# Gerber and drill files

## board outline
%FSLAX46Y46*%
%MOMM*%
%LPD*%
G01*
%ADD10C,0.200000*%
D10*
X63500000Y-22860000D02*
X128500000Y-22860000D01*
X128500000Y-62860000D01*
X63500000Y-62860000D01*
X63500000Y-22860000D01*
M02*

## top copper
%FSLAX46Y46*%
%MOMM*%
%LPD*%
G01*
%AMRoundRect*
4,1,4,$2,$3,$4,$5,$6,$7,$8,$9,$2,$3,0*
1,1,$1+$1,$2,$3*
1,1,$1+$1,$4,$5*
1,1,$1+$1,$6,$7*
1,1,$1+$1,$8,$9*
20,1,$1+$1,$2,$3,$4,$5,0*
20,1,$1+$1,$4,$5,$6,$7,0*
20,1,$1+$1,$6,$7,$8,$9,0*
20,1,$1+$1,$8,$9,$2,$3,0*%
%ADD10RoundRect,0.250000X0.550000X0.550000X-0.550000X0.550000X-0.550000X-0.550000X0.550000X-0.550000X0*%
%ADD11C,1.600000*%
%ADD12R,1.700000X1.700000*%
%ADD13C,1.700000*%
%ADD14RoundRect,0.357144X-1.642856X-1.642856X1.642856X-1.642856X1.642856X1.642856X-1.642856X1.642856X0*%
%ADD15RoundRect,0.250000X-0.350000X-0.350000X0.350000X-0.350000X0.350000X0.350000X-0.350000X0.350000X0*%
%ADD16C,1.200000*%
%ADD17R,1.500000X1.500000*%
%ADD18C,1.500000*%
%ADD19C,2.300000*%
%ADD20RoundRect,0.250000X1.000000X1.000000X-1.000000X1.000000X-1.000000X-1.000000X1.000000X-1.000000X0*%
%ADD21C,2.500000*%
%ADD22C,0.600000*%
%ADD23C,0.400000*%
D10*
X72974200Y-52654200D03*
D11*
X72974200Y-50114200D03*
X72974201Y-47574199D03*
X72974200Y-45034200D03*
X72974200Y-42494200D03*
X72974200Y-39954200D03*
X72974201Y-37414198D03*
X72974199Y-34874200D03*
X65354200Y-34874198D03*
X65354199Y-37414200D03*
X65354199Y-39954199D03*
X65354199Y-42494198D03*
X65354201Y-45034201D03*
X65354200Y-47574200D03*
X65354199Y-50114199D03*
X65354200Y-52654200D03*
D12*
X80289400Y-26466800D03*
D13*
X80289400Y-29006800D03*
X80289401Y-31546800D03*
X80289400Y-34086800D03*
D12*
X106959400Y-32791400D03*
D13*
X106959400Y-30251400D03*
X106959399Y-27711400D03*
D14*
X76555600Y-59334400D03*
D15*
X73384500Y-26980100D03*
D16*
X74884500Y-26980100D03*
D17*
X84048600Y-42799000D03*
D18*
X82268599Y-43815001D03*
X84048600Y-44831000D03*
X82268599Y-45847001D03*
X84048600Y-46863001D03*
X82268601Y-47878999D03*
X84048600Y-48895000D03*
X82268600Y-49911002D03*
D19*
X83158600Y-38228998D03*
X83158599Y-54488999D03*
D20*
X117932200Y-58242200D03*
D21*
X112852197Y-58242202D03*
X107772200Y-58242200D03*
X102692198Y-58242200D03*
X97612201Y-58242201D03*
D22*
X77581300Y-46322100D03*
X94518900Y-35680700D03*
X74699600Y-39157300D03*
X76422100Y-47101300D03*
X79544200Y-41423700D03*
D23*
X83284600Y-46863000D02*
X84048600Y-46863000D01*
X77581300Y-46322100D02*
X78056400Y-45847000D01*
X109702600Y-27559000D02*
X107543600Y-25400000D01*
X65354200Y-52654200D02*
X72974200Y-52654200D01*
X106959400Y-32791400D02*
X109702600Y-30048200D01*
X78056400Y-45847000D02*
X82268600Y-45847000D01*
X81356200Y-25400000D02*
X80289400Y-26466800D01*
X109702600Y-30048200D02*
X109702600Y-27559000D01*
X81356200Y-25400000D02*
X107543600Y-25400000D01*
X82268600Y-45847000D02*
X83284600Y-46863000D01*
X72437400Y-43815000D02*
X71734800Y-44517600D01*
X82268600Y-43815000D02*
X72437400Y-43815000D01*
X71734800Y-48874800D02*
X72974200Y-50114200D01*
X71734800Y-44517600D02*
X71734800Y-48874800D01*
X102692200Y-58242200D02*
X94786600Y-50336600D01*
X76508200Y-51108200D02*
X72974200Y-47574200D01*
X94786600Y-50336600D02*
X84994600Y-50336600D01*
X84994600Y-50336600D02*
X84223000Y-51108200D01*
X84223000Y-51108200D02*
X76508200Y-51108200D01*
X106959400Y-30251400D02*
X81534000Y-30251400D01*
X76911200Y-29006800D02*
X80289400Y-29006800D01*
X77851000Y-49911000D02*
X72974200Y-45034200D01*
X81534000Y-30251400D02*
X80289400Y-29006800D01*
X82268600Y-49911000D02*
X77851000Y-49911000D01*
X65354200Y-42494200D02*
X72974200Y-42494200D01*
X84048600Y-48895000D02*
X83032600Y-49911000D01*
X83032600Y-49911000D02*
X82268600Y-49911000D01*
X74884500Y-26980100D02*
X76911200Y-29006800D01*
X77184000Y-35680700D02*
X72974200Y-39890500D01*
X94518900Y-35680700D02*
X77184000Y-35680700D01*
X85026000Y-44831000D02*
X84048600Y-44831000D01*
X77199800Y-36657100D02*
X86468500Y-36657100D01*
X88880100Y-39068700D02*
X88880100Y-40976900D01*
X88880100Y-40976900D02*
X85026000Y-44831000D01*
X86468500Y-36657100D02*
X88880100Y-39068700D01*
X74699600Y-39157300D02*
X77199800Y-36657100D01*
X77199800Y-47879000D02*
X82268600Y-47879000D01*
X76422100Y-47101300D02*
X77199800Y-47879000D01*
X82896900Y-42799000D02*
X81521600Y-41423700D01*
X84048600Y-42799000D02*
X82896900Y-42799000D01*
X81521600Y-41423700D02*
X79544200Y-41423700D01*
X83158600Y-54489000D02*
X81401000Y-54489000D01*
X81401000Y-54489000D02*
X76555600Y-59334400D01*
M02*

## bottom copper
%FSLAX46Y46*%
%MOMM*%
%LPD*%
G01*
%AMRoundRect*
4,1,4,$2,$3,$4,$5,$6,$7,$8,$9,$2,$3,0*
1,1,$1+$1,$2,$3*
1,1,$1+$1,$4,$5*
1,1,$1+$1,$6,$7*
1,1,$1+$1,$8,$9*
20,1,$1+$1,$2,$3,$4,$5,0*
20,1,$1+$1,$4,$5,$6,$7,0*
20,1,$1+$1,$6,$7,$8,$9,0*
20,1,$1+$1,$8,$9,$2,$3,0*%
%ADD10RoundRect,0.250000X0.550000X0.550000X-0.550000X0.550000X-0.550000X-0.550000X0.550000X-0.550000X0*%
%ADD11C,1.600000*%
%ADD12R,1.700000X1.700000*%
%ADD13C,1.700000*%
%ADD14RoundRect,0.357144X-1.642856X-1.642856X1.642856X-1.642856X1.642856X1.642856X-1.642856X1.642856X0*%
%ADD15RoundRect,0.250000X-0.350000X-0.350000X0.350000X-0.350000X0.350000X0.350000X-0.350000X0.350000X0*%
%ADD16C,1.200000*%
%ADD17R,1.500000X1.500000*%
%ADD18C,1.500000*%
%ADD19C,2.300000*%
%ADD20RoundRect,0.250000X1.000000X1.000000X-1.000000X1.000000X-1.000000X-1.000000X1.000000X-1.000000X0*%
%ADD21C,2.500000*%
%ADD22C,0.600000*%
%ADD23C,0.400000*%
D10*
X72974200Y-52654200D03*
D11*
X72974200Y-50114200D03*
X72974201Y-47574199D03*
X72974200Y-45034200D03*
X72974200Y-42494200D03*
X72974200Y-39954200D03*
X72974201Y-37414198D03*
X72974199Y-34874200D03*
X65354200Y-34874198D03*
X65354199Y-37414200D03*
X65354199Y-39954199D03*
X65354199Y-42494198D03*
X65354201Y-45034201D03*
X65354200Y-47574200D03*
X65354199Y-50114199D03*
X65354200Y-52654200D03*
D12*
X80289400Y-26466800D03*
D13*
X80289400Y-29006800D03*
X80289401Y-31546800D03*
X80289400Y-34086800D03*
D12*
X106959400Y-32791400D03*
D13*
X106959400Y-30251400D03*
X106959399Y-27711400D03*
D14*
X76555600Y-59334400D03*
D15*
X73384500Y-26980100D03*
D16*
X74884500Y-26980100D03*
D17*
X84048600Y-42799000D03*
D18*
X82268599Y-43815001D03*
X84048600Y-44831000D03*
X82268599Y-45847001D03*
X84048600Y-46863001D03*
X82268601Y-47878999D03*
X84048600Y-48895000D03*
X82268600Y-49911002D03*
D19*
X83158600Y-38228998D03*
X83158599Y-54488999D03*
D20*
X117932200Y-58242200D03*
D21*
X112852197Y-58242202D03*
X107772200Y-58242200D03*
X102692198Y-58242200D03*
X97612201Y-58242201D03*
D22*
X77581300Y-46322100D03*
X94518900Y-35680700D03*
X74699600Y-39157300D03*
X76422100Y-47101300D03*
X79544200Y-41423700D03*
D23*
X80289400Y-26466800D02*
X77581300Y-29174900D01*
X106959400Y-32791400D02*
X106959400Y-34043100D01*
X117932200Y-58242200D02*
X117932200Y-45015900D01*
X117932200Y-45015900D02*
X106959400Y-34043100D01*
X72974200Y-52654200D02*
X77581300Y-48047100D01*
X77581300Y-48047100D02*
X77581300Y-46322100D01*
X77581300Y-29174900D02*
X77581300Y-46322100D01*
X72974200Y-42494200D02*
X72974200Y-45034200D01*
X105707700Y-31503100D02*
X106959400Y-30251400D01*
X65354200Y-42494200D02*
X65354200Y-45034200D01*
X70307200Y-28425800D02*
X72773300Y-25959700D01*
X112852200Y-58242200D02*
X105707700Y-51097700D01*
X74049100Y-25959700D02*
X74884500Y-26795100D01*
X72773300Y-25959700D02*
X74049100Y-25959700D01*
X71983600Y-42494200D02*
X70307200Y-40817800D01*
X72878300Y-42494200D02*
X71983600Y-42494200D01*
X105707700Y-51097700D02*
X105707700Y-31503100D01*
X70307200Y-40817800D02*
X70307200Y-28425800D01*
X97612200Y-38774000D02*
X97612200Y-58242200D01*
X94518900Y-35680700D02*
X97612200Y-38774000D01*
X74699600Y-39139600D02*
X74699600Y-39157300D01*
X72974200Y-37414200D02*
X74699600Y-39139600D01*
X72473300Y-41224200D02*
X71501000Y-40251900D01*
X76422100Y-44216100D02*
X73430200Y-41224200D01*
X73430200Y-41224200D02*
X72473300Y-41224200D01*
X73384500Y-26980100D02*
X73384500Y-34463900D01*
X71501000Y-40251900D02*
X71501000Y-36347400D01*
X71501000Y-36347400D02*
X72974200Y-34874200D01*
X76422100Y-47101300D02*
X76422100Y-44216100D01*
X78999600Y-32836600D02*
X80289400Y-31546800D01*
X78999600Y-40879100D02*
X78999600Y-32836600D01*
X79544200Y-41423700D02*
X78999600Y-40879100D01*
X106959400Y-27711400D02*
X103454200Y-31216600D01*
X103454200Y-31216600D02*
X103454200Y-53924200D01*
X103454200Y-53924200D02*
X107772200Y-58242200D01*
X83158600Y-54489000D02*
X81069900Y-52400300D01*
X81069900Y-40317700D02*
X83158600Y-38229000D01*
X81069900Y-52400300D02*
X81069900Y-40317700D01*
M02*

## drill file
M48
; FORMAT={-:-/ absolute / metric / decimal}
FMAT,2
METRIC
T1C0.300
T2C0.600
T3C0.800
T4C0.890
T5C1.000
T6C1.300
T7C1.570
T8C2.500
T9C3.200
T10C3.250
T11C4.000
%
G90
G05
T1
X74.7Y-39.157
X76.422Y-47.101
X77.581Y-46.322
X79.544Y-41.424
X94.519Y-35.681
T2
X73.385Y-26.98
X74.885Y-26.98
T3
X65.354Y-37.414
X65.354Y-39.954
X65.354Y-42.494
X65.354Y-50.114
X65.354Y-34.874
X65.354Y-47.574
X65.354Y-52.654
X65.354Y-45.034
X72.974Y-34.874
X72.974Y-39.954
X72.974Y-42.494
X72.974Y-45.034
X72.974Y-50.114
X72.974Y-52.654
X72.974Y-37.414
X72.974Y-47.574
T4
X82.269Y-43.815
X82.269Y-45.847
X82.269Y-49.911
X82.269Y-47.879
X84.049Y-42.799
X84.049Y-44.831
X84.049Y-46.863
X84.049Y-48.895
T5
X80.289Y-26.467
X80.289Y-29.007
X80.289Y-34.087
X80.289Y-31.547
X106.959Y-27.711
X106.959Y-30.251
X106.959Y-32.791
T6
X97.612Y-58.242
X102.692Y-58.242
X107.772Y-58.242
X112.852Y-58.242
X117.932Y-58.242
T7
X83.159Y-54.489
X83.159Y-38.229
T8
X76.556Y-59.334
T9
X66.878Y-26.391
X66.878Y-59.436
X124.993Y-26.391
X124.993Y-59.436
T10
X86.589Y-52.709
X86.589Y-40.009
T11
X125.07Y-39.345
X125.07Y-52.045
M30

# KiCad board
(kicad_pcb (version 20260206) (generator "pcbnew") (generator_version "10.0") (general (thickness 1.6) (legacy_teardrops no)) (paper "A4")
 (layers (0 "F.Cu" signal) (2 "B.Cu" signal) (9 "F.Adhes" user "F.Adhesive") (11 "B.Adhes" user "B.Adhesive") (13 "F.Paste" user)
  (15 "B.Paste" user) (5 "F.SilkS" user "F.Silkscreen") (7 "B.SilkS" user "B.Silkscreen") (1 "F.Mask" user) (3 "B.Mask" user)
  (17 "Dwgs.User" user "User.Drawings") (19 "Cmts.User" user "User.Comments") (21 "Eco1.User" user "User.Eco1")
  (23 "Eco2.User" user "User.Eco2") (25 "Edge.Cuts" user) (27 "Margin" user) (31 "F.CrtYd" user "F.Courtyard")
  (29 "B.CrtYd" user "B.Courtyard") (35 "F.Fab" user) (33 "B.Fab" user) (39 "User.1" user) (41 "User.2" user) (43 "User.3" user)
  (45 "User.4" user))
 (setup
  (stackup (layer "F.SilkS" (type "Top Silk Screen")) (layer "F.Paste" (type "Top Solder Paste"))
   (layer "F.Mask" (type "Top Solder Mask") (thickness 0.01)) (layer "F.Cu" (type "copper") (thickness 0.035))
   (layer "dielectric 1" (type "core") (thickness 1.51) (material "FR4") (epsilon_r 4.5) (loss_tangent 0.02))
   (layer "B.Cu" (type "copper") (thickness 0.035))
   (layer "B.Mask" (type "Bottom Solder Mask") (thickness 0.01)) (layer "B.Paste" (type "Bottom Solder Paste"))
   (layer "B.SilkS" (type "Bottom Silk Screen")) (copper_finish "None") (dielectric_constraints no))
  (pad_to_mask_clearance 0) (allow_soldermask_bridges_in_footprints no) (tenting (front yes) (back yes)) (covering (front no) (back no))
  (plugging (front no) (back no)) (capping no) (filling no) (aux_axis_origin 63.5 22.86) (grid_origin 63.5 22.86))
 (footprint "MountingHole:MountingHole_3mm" (layer "F.Cu") (at 125.0696 52.0446)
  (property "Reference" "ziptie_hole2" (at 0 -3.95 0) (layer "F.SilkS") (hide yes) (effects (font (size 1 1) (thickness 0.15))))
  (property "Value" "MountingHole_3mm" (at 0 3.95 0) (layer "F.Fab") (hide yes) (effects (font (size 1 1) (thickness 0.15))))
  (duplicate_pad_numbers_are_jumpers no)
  (pad "" np_thru_hole circle (at 0 0) (size 4 4) (drill 4) (layers "*.Cu" "*.Mask")))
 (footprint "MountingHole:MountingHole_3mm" (layer "F.Cu") (at 125.0696 39.3446)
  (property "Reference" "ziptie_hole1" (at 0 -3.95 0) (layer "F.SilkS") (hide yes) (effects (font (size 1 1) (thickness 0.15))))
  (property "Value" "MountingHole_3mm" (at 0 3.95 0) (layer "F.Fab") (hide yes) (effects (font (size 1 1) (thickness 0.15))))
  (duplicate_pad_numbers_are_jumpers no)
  (pad "" np_thru_hole circle (at 0 0) (size 4 4) (drill 4) (layers "*.Cu" "*.Mask")))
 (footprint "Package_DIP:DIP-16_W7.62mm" (layer "F.Cu") (at 72.9742 52.6542 180)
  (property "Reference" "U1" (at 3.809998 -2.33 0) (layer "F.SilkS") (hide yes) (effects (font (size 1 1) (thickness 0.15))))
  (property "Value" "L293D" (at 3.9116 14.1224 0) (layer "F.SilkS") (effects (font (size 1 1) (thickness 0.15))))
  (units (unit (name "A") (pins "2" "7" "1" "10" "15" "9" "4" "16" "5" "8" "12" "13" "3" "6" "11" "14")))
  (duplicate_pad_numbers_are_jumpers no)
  (pad "1" thru_hole roundrect (at 0 0 180) (size 1.6 1.6) (drill 0.8) (layers "*.Cu" "*.Mask") (remove_unused_layers no)
   (roundrect_rratio 0.15625) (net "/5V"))
  (pad "2" thru_hole circle (at 0 2.54 180) (size 1.6 1.6) (drill 0.8) (layers "*.Cu" "*.Mask") (remove_unused_layers no) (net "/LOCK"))
  (pad "3" thru_hole circle (at -0.000001 5.080001 180) (size 1.6 1.6) (drill 0.8) (layers "*.Cu" "*.Mask") (remove_unused_layers no)
   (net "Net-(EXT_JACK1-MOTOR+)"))
  (pad "4" thru_hole circle (at 0 7.62 180) (size 1.6 1.6) (drill 0.8) (layers "*.Cu" "*.Mask") (remove_unused_layers no) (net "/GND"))
  (pad "5" thru_hole circle (at 0 10.16 180) (size 1.6 1.6) (drill 0.8) (layers "*.Cu" "*.Mask") (remove_unused_layers no) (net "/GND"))
  (pad "6" thru_hole circle (at 0 12.7 180) (size 1.6 1.6) (drill 0.8) (layers "*.Cu" "*.Mask") (remove_unused_layers no)
   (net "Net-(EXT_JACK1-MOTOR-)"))
  (pad "7" thru_hole circle (at -0.000001 15.240002 180) (size 1.6 1.6) (drill 0.8) (layers "*.Cu" "*.Mask") (remove_unused_layers no)
   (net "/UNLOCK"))
  (pad "8" thru_hole circle (at 0.000001 17.78 180) (size 1.6 1.6) (drill 0.8) (layers "*.Cu" "*.Mask") (remove_unused_layers no)
   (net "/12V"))
  (pad "9" thru_hole circle (at 7.62 17.780002 180) (size 1.6 1.6) (drill 0.8) (layers "*.Cu" "*.Mask") (remove_unused_layers no)
   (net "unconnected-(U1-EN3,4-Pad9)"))
  (pad "10" thru_hole circle (at 7.620001 15.24 180) (size 1.6 1.6) (drill 0.8) (layers "*.Cu" "*.Mask") (remove_unused_layers no)
   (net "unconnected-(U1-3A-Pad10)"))
  (pad "11" thru_hole circle (at 7.620001 12.700001 180) (size 1.6 1.6) (drill 0.8) (layers "*.Cu" "*.Mask") (remove_unused_layers no)
   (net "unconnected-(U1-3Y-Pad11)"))
  (pad "12" thru_hole circle (at 7.620001 10.160002 180) (size 1.6 1.6) (drill 0.8) (layers "*.Cu" "*.Mask") (remove_unused_layers no)
   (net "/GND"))
  (pad "13" thru_hole circle (at 7.619999 7.619999 180) (size 1.6 1.6) (drill 0.8) (layers "*.Cu" "*.Mask") (remove_unused_layers no)
   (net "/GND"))
  (pad "14" thru_hole circle (at 7.62 5.08 180) (size 1.6 1.6) (drill 0.8) (layers "*.Cu" "*.Mask") (remove_unused_layers no)
   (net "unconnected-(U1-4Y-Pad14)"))
  (pad "15" thru_hole circle (at 7.620001 2.540001 180) (size 1.6 1.6) (drill 0.8) (layers "*.Cu" "*.Mask") (remove_unused_layers no)
   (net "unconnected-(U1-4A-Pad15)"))
  (pad "16" thru_hole circle (at 7.62 0 180) (size 1.6 1.6) (drill 0.8) (layers "*.Cu" "*.Mask") (remove_unused_layers no) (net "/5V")))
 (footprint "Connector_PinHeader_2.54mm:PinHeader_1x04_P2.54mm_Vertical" (layer "F.Cu") (at 80.2894 26.4668)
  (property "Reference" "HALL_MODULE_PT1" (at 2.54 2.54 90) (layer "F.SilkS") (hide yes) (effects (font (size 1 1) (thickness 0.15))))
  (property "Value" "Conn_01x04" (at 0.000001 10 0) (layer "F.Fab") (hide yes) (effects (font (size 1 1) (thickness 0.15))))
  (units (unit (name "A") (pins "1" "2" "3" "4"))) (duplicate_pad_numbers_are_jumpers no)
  (pad "1" thru_hole rect (at 0 0) (size 1.7 1.7) (drill 1) (layers "*.Cu" "*.Mask") (remove_unused_layers no) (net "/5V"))
  (pad "2" thru_hole circle (at 0 2.54) (size 1.7 1.7) (drill 1) (layers "*.Cu" "*.Mask") (remove_unused_layers no) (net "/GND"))
  (pad "3" thru_hole circle (at 0.000001 5.08) (size 1.7 1.7) (drill 1) (layers "*.Cu" "*.Mask") (remove_unused_layers no) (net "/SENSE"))
  (pad "4" thru_hole circle (at 0 7.62) (size 1.7 1.7) (drill 1) (layers "*.Cu" "*.Mask") (remove_unused_layers no)
   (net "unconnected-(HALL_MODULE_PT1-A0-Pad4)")))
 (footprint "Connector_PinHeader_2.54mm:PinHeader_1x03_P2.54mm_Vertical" (layer "F.Cu") (at 106.9594 32.7914 180)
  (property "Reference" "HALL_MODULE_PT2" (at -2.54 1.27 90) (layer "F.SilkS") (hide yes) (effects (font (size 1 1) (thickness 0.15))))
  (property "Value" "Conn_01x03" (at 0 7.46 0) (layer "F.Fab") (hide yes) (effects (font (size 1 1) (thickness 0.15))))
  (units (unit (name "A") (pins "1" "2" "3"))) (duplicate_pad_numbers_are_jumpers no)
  (pad "1" thru_hole rect (at 0 0 180) (size 1.7 1.7) (drill 1) (layers "*.Cu" "*.Mask") (remove_unused_layers no) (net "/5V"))
  (pad "2" thru_hole circle (at 0 2.54 180) (size 1.7 1.7) (drill 1) (layers "*.Cu" "*.Mask") (remove_unused_layers no) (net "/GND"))
  (pad "3" thru_hole circle (at 0.000001 5.08 180) (size 1.7 1.7) (drill 1) (layers "*.Cu" "*.Mask") (remove_unused_layers no) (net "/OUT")))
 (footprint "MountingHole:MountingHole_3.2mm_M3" (layer "F.Cu") (at 124.9934 26.3906)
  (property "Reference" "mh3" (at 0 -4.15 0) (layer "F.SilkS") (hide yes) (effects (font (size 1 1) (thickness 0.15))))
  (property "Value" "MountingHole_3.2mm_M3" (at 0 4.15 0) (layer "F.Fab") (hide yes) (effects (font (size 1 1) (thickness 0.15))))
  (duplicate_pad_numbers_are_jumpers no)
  (pad "" np_thru_hole circle (at 0 0) (size 3.2 3.2) (drill 3.2) (layers "*.Cu" "*.Mask")))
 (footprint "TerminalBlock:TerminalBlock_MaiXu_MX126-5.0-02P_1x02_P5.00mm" (layer "F.Cu") (at 76.5556 59.3344)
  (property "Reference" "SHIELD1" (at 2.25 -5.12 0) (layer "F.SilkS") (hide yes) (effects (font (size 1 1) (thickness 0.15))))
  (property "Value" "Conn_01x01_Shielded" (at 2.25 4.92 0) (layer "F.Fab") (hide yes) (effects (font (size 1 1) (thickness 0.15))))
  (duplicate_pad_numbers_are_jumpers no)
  (pad "1" thru_hole roundrect (at 0 0) (size 4 4) (drill 2.5) (layers "*.Cu" "*.Mask") (remove_unused_layers no)
   (roundrect_rratio 0.089286) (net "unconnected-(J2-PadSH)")))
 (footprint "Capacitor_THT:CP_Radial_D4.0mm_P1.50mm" (layer "F.Cu") (at 73.3845 26.9801)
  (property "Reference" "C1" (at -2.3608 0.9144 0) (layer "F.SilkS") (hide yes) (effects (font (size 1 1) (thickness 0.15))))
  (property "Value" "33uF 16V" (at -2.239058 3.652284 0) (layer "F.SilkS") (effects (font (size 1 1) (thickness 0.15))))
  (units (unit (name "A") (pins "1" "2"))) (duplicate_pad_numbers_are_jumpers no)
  (pad "1" thru_hole roundrect (at 0 0) (size 1.2 1.2) (drill 0.6) (layers "*.Cu" "*.Mask") (remove_unused_layers no)
   (roundrect_rratio 0.208333) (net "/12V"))
  (pad "2" thru_hole circle (at 1.5 0) (size 1.2 1.2) (drill 0.6) (layers "*.Cu" "*.Mask") (remove_unused_layers no) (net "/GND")))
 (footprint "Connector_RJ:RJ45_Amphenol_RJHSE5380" (layer "F.Cu") (at 84.0486 42.799 -90)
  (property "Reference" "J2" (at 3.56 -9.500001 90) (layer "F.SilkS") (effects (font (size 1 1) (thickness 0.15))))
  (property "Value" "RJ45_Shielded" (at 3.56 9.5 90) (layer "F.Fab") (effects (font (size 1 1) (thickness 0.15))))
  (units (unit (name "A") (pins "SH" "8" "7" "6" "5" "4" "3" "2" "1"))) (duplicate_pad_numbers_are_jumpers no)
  (pad "" np_thru_hole circle (at -2.79 -2.54 270) (size 3.25 3.25) (drill 3.25) (layers "*.Cu" "*.Mask"))
  (pad "" np_thru_hole circle (at 9.909999 -2.539999 270) (size 3.25 3.25) (drill 3.25) (layers "*.Cu" "*.Mask"))
  (pad "1" thru_hole rect (at 0 0 270) (size 1.5 1.5) (drill 0.89) (layers "*.Cu" "*.Mask") (remove_unused_layers no) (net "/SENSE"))
  (pad "2" thru_hole circle (at 1.016001 1.780001 270) (size 1.5 1.5) (drill 0.89) (layers "*.Cu" "*.Mask") (remove_unused_layers no)
   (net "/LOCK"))
  (pad "3" thru_hole circle (at 2.032 0 270) (size 1.5 1.5) (drill 0.89) (layers "*.Cu" "*.Mask") (remove_unused_layers no) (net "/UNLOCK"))
  (pad "4" thru_hole circle (at 3.048001 1.780001 270) (size 1.5 1.5) (drill 0.89) (layers "*.Cu" "*.Mask") (remove_unused_layers no)
   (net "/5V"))
  (pad "5" thru_hole circle (at 4.064001 0 270) (size 1.5 1.5) (drill 0.89) (layers "*.Cu" "*.Mask") (remove_unused_layers no) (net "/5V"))
  (pad "6" thru_hole circle (at 5.079999 1.779999 270) (size 1.5 1.5) (drill 0.89) (layers "*.Cu" "*.Mask") (remove_unused_layers no)
   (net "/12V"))
  (pad "7" thru_hole circle (at 6.096 0 270) (size 1.5 1.5) (drill 0.89) (layers "*.Cu" "*.Mask") (remove_unused_layers no) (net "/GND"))
  (pad "8" thru_hole circle (at 7.112002 1.78 270) (size 1.5 1.5) (drill 0.89) (layers "*.Cu" "*.Mask") (remove_unused_layers no)
   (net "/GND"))
  (pad "SH" thru_hole circle (at -4.570002 0.89 270) (size 2.3 2.3) (drill 1.57) (layers "*.Cu" "*.Mask") (remove_unused_layers no)
   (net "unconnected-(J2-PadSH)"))
  (pad "SH" thru_hole circle (at 11.689999 0.890001 270) (size 2.3 2.3) (drill 1.57) (layers "*.Cu" "*.Mask") (remove_unused_layers no)
   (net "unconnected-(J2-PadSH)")))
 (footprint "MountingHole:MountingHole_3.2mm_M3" (layer "F.Cu") (at 66.8782 59.436)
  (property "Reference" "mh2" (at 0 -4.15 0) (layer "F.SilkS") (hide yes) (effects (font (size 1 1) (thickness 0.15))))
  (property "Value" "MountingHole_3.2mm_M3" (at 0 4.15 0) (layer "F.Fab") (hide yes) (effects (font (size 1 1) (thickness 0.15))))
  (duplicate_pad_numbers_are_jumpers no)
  (pad "" np_thru_hole circle (at 0 0) (size 3.2 3.2) (drill 3.2) (layers "*.Cu" "*.Mask")))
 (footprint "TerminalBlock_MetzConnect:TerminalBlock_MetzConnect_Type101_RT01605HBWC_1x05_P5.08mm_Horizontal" (layer "F.Cu")
  (at 117.9322 58.2422 180)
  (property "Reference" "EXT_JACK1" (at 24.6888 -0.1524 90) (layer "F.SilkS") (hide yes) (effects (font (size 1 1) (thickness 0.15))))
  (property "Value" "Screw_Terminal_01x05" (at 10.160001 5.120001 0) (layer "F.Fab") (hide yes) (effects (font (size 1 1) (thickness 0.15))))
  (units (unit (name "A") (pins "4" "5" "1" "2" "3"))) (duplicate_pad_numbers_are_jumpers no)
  (pad "1" thru_hole roundrect (at 0 0 180) (size 2.5 2.5) (drill 1.3) (layers "*.Cu" "*.Mask") (remove_unused_layers no)
   (roundrect_rratio 0.1) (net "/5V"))
  (pad "2" thru_hole circle (at 5.080003 -0.000002 180) (size 2.5 2.5) (drill 1.3) (layers "*.Cu" "*.Mask") (remove_unused_layers no)
   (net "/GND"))
  (pad "3" thru_hole circle (at 10.16 0 180) (size 2.5 2.5) (drill 1.3) (layers "*.Cu" "*.Mask") (remove_unused_layers no) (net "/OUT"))
  (pad "4" thru_hole circle (at 15.240002 0 180) (size 2.5 2.5) (drill 1.3) (layers "*.Cu" "*.Mask") (remove_unused_layers no)
   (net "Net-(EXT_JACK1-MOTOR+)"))
  (pad "5" thru_hole circle (at 20.319999 -0.000001 180) (size 2.5 2.5) (drill 1.3) (layers "*.Cu" "*.Mask") (remove_unused_layers no)
   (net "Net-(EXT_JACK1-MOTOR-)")))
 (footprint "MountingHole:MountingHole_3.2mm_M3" (layer "F.Cu") (at 66.8782 26.3906)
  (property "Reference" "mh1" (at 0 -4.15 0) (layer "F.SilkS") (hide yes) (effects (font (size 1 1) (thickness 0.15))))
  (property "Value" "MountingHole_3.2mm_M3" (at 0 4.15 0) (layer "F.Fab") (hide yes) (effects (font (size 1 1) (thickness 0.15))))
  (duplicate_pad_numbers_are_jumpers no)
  (pad "" np_thru_hole circle (at 0 0) (size 3.2 3.2) (drill 3.2) (layers "*.Cu" "*.Mask")))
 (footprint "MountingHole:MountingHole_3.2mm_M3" (layer "F.Cu") (at 124.9934 59.436)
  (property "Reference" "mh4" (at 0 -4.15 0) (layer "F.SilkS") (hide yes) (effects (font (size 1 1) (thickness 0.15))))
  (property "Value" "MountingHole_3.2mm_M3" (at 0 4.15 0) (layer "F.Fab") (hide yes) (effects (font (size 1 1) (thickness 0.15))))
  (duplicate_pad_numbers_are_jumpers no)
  (pad "" np_thru_hole circle (at 0 0) (size 3.2 3.2) (drill 3.2) (layers "*.Cu" "*.Mask")))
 (gr_rect (start 63.5 22.86) (end 128.5 62.86) (stroke (width 0.2) (type solid)) (fill no) (layer "Edge.Cuts"))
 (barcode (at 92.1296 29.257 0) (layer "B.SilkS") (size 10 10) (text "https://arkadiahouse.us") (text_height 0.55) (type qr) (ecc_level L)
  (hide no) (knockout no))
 (segment (start 83.2846 46.863) (end 84.0486 46.863) (width 0.4) (layer "F.Cu") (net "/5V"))
 (segment (start 77.5813 46.3221) (end 78.0564 45.847) (width 0.4) (layer "F.Cu") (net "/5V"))
 (segment (start 109.7026 27.559) (end 107.5436 25.4) (width 0.4) (layer "F.Cu") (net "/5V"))
 (segment (start 65.3542 52.6542) (end 72.9742 52.6542) (width 0.4) (layer "F.Cu") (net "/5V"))
 (segment (start 106.9594 32.7914) (end 109.7026 30.0482) (width 0.4) (layer "F.Cu") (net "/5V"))
 (segment (start 78.0564 45.847) (end 82.2686 45.847) (width 0.4) (layer "F.Cu") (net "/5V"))
 (segment (start 81.3562 25.4) (end 80.2894 26.4668) (width 0.4) (layer "F.Cu") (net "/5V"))
 (segment (start 109.7026 30.0482) (end 109.7026 27.559) (width 0.4) (layer "F.Cu") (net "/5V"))
 (segment (start 81.3562 25.4) (end 107.5436 25.4) (width 0.4) (layer "F.Cu") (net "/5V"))
 (segment (start 82.2686 45.847) (end 83.2846 46.863) (width 0.4) (layer "F.Cu") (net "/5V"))
 (via (at 77.5813 46.3221) (size 0.6) (drill 0.3) (layers "F.Cu" "B.Cu") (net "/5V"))
 (segment (start 80.2894 26.4668) (end 77.5813 29.1749) (width 0.4) (layer "B.Cu") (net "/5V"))
 (segment (start 106.9594 32.7914) (end 106.9594 34.0431) (width 0.4) (layer "B.Cu") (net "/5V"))
 (segment (start 117.9322 58.2422) (end 117.9322 45.0159) (width 0.4) (layer "B.Cu") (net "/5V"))
 (segment (start 117.9322 45.0159) (end 106.9594 34.0431) (width 0.4) (layer "B.Cu") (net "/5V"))
 (segment (start 72.9742 52.6542) (end 77.5813 48.0471) (width 0.4) (layer "B.Cu") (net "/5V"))
 (segment (start 77.5813 48.0471) (end 77.5813 46.3221) (width 0.4) (layer "B.Cu") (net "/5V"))
 (segment (start 77.5813 29.1749) (end 77.5813 46.3221) (width 0.4) (layer "B.Cu") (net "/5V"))
 (segment (start 72.4374 43.815) (end 71.7348 44.5176) (width 0.4) (layer "F.Cu") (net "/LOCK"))
 (segment (start 82.2686 43.815) (end 72.4374 43.815) (width 0.4) (layer "F.Cu") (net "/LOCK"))
 (segment (start 71.7348 48.8748) (end 72.9742 50.1142) (width 0.4) (layer "F.Cu") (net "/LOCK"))
 (segment (start 71.7348 44.5176) (end 71.7348 48.8748) (width 0.4) (layer "F.Cu") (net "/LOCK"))
 (segment (start 102.6922 58.2422) (end 94.7866 50.3366) (width 0.4) (layer "F.Cu") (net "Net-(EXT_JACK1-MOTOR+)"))
 (segment (start 76.5082 51.1082) (end 72.9742 47.5742) (width 0.4) (layer "F.Cu") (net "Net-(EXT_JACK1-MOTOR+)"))
 (segment (start 94.7866 50.3366) (end 84.9946 50.3366) (width 0.4) (layer "F.Cu") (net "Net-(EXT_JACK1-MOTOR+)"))
 (segment (start 84.9946 50.3366) (end 84.223 51.1082) (width 0.4) (layer "F.Cu") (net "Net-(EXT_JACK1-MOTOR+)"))
 (segment (start 84.223 51.1082) (end 76.5082 51.1082) (width 0.4) (layer "F.Cu") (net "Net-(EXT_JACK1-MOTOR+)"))
 (segment (start 106.9594 30.2514) (end 81.534 30.2514) (width 0.4) (layer "F.Cu") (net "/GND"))
 (segment (start 76.9112 29.0068) (end 80.2894 29.0068) (width 0.4) (layer "F.Cu") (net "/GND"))
 (segment (start 77.851 49.911) (end 72.9742 45.0342) (width 0.4) (layer "F.Cu") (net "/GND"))
 (segment (start 81.534 30.2514) (end 80.2894 29.0068) (width 0.4) (layer "F.Cu") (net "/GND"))
 (segment (start 82.2686 49.911) (end 77.851 49.911) (width 0.4) (layer "F.Cu") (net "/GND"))
 (segment (start 65.3542 42.4942) (end 72.9742 42.4942) (width 0.4) (layer "F.Cu") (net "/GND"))
 (segment (start 84.0486 48.895) (end 83.0326 49.911) (width 0.4) (layer "F.Cu") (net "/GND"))
 (segment (start 83.0326 49.911) (end 82.2686 49.911) (width 0.4) (layer "F.Cu") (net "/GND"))
 (segment (start 74.8845 26.9801) (end 76.9112 29.0068) (width 0.4) (layer "F.Cu") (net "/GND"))
 (segment (start 72.9742 42.4942) (end 72.9742 45.0342) (width 0.4) (layer "B.Cu") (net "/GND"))
 (segment (start 105.7077 31.5031) (end 106.9594 30.2514) (width 0.4) (layer "B.Cu") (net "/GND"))
 (segment (start 65.3542 42.4942) (end 65.3542 45.0342) (width 0.4) (layer "B.Cu") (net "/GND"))
 (segment (start 70.3072 28.4258) (end 72.7733 25.9597) (width 0.4) (layer "B.Cu") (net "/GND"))
 (segment (start 112.8522 58.2422) (end 105.7077 51.0977) (width 0.4) (layer "B.Cu") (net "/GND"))
 (segment (start 74.0491 25.9597) (end 74.8845 26.7951) (width 0.4) (layer "B.Cu") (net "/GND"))
 (segment (start 72.7733 25.9597) (end 74.0491 25.9597) (width 0.4) (layer "B.Cu") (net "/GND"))
 (segment (start 71.9836 42.4942) (end 70.3072 40.8178) (width 0.4) (layer "B.Cu") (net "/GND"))
 (segment (start 72.8783 42.4942) (end 71.9836 42.4942) (width 0.4) (layer "B.Cu") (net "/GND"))
 (segment (start 105.7077 51.0977) (end 105.7077 31.5031) (width 0.4) (layer "B.Cu") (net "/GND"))
 (segment (start 70.3072 40.8178) (end 70.3072 28.4258) (width 0.4) (layer "B.Cu") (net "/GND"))
 (segment (start 77.184 35.6807) (end 72.9742 39.8905) (width 0.4) (layer "F.Cu") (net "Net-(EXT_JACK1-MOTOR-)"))
 (segment (start 94.5189 35.6807) (end 77.184 35.6807) (width 0.4) (layer "F.Cu") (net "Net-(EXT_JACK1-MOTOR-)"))
 (via (at 94.5189 35.6807) (size 0.6) (drill 0.3) (layers "F.Cu" "B.Cu") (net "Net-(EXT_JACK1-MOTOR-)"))
 (segment (start 97.6122 38.774) (end 97.6122 58.2422) (width 0.4) (layer "B.Cu") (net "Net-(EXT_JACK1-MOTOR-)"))
 (segment (start 94.5189 35.6807) (end 97.6122 38.774) (width 0.4) (layer "B.Cu") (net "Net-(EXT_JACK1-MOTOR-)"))
 (segment (start 85.026 44.831) (end 84.0486 44.831) (width 0.4) (layer "F.Cu") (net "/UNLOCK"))
 (segment (start 77.1998 36.6571) (end 86.4685 36.6571) (width 0.4) (layer "F.Cu") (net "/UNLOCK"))
 (segment (start 88.8801 39.0687) (end 88.8801 40.9769) (width 0.4) (layer "F.Cu") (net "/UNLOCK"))
 (segment (start 88.8801 40.9769) (end 85.026 44.831) (width 0.4) (layer "F.Cu") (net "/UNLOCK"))
 (segment (start 86.4685 36.6571) (end 88.8801 39.0687) (width 0.4) (layer "F.Cu") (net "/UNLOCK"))
 (segment (start 74.6996 39.1573) (end 77.1998 36.6571) (width 0.4) (layer "F.Cu") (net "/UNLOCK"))
 (via (at 74.6996 39.1573) (size 0.6) (drill 0.3) (layers "F.Cu" "B.Cu") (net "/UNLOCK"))
 (segment (start 74.6996 39.1396) (end 74.6996 39.1573) (width 0.4) (layer "B.Cu") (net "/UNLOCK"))
 (segment (start 72.9742 37.4142) (end 74.6996 39.1396) (width 0.4) (layer "B.Cu") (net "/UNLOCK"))
 (segment (start 77.1998 47.879) (end 82.2686 47.879) (width 0.4) (layer "F.Cu") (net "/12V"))
 (segment (start 76.4221 47.1013) (end 77.1998 47.879) (width 0.4) (layer "F.Cu") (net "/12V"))
 (via (at 76.4221 47.1013) (size 0.6) (drill 0.3) (layers "F.Cu" "B.Cu") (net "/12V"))
 (segment (start 72.4733 41.2242) (end 71.501 40.2519) (width 0.4) (layer "B.Cu") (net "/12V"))
 (segment (start 76.4221 44.2161) (end 73.4302 41.2242) (width 0.4) (layer "B.Cu") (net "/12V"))
 (segment (start 73.4302 41.2242) (end 72.4733 41.2242) (width 0.4) (layer "B.Cu") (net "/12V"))
 (segment (start 73.3845 26.9801) (end 73.3845 34.4639) (width 0.4) (layer "B.Cu") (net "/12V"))
 (segment (start 71.501 40.2519) (end 71.501 36.3474) (width 0.4) (layer "B.Cu") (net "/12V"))
 (segment (start 71.501 36.3474) (end 72.9742 34.8742) (width 0.4) (layer "B.Cu") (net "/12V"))
 (segment (start 76.4221 47.1013) (end 76.4221 44.2161) (width 0.4) (layer "B.Cu") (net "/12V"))
 (segment (start 82.8969 42.799) (end 81.5216 41.4237) (width 0.4) (layer "F.Cu") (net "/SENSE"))
 (segment (start 84.0486 42.799) (end 82.8969 42.799) (width 0.4) (layer "F.Cu") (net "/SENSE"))
 (segment (start 81.5216 41.4237) (end 79.5442 41.4237) (width 0.4) (layer "F.Cu") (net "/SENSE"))
 (via (at 79.5442 41.4237) (size 0.6) (drill 0.3) (layers "F.Cu" "B.Cu") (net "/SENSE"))
 (segment (start 78.9996 32.8366) (end 80.2894 31.5468) (width 0.4) (layer "B.Cu") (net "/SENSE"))
 (segment (start 78.9996 40.8791) (end 78.9996 32.8366) (width 0.4) (layer "B.Cu") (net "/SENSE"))
 (segment (start 79.5442 41.4237) (end 78.9996 40.8791) (width 0.4) (layer "B.Cu") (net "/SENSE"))
 (segment (start 106.9594 27.7114) (end 103.4542 31.2166) (width 0.4) (layer "B.Cu") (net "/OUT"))
 (segment (start 103.4542 31.2166) (end 103.4542 53.9242) (width 0.4) (layer "B.Cu") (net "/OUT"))
 (segment (start 103.4542 53.9242) (end 107.7722 58.2422) (width 0.4) (layer "B.Cu") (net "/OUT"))
 (segment (start 83.1586 54.489) (end 81.401 54.489) (width 0.4) (layer "F.Cu") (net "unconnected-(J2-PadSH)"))
 (segment (start 81.401 54.489) (end 76.5556 59.3344) (width 0.4) (layer "F.Cu") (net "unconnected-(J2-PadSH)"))
 (segment (start 83.1586 54.489) (end 81.0699 52.4003) (width 0.4) (layer "B.Cu") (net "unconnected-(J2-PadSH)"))
 (segment (start 81.0699 40.3177) (end 83.1586 38.229) (width 0.4) (layer "B.Cu") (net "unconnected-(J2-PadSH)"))
 (segment (start 81.0699 52.4003) (end 81.0699 40.3177) (width 0.4) (layer "B.Cu") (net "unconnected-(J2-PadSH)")))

